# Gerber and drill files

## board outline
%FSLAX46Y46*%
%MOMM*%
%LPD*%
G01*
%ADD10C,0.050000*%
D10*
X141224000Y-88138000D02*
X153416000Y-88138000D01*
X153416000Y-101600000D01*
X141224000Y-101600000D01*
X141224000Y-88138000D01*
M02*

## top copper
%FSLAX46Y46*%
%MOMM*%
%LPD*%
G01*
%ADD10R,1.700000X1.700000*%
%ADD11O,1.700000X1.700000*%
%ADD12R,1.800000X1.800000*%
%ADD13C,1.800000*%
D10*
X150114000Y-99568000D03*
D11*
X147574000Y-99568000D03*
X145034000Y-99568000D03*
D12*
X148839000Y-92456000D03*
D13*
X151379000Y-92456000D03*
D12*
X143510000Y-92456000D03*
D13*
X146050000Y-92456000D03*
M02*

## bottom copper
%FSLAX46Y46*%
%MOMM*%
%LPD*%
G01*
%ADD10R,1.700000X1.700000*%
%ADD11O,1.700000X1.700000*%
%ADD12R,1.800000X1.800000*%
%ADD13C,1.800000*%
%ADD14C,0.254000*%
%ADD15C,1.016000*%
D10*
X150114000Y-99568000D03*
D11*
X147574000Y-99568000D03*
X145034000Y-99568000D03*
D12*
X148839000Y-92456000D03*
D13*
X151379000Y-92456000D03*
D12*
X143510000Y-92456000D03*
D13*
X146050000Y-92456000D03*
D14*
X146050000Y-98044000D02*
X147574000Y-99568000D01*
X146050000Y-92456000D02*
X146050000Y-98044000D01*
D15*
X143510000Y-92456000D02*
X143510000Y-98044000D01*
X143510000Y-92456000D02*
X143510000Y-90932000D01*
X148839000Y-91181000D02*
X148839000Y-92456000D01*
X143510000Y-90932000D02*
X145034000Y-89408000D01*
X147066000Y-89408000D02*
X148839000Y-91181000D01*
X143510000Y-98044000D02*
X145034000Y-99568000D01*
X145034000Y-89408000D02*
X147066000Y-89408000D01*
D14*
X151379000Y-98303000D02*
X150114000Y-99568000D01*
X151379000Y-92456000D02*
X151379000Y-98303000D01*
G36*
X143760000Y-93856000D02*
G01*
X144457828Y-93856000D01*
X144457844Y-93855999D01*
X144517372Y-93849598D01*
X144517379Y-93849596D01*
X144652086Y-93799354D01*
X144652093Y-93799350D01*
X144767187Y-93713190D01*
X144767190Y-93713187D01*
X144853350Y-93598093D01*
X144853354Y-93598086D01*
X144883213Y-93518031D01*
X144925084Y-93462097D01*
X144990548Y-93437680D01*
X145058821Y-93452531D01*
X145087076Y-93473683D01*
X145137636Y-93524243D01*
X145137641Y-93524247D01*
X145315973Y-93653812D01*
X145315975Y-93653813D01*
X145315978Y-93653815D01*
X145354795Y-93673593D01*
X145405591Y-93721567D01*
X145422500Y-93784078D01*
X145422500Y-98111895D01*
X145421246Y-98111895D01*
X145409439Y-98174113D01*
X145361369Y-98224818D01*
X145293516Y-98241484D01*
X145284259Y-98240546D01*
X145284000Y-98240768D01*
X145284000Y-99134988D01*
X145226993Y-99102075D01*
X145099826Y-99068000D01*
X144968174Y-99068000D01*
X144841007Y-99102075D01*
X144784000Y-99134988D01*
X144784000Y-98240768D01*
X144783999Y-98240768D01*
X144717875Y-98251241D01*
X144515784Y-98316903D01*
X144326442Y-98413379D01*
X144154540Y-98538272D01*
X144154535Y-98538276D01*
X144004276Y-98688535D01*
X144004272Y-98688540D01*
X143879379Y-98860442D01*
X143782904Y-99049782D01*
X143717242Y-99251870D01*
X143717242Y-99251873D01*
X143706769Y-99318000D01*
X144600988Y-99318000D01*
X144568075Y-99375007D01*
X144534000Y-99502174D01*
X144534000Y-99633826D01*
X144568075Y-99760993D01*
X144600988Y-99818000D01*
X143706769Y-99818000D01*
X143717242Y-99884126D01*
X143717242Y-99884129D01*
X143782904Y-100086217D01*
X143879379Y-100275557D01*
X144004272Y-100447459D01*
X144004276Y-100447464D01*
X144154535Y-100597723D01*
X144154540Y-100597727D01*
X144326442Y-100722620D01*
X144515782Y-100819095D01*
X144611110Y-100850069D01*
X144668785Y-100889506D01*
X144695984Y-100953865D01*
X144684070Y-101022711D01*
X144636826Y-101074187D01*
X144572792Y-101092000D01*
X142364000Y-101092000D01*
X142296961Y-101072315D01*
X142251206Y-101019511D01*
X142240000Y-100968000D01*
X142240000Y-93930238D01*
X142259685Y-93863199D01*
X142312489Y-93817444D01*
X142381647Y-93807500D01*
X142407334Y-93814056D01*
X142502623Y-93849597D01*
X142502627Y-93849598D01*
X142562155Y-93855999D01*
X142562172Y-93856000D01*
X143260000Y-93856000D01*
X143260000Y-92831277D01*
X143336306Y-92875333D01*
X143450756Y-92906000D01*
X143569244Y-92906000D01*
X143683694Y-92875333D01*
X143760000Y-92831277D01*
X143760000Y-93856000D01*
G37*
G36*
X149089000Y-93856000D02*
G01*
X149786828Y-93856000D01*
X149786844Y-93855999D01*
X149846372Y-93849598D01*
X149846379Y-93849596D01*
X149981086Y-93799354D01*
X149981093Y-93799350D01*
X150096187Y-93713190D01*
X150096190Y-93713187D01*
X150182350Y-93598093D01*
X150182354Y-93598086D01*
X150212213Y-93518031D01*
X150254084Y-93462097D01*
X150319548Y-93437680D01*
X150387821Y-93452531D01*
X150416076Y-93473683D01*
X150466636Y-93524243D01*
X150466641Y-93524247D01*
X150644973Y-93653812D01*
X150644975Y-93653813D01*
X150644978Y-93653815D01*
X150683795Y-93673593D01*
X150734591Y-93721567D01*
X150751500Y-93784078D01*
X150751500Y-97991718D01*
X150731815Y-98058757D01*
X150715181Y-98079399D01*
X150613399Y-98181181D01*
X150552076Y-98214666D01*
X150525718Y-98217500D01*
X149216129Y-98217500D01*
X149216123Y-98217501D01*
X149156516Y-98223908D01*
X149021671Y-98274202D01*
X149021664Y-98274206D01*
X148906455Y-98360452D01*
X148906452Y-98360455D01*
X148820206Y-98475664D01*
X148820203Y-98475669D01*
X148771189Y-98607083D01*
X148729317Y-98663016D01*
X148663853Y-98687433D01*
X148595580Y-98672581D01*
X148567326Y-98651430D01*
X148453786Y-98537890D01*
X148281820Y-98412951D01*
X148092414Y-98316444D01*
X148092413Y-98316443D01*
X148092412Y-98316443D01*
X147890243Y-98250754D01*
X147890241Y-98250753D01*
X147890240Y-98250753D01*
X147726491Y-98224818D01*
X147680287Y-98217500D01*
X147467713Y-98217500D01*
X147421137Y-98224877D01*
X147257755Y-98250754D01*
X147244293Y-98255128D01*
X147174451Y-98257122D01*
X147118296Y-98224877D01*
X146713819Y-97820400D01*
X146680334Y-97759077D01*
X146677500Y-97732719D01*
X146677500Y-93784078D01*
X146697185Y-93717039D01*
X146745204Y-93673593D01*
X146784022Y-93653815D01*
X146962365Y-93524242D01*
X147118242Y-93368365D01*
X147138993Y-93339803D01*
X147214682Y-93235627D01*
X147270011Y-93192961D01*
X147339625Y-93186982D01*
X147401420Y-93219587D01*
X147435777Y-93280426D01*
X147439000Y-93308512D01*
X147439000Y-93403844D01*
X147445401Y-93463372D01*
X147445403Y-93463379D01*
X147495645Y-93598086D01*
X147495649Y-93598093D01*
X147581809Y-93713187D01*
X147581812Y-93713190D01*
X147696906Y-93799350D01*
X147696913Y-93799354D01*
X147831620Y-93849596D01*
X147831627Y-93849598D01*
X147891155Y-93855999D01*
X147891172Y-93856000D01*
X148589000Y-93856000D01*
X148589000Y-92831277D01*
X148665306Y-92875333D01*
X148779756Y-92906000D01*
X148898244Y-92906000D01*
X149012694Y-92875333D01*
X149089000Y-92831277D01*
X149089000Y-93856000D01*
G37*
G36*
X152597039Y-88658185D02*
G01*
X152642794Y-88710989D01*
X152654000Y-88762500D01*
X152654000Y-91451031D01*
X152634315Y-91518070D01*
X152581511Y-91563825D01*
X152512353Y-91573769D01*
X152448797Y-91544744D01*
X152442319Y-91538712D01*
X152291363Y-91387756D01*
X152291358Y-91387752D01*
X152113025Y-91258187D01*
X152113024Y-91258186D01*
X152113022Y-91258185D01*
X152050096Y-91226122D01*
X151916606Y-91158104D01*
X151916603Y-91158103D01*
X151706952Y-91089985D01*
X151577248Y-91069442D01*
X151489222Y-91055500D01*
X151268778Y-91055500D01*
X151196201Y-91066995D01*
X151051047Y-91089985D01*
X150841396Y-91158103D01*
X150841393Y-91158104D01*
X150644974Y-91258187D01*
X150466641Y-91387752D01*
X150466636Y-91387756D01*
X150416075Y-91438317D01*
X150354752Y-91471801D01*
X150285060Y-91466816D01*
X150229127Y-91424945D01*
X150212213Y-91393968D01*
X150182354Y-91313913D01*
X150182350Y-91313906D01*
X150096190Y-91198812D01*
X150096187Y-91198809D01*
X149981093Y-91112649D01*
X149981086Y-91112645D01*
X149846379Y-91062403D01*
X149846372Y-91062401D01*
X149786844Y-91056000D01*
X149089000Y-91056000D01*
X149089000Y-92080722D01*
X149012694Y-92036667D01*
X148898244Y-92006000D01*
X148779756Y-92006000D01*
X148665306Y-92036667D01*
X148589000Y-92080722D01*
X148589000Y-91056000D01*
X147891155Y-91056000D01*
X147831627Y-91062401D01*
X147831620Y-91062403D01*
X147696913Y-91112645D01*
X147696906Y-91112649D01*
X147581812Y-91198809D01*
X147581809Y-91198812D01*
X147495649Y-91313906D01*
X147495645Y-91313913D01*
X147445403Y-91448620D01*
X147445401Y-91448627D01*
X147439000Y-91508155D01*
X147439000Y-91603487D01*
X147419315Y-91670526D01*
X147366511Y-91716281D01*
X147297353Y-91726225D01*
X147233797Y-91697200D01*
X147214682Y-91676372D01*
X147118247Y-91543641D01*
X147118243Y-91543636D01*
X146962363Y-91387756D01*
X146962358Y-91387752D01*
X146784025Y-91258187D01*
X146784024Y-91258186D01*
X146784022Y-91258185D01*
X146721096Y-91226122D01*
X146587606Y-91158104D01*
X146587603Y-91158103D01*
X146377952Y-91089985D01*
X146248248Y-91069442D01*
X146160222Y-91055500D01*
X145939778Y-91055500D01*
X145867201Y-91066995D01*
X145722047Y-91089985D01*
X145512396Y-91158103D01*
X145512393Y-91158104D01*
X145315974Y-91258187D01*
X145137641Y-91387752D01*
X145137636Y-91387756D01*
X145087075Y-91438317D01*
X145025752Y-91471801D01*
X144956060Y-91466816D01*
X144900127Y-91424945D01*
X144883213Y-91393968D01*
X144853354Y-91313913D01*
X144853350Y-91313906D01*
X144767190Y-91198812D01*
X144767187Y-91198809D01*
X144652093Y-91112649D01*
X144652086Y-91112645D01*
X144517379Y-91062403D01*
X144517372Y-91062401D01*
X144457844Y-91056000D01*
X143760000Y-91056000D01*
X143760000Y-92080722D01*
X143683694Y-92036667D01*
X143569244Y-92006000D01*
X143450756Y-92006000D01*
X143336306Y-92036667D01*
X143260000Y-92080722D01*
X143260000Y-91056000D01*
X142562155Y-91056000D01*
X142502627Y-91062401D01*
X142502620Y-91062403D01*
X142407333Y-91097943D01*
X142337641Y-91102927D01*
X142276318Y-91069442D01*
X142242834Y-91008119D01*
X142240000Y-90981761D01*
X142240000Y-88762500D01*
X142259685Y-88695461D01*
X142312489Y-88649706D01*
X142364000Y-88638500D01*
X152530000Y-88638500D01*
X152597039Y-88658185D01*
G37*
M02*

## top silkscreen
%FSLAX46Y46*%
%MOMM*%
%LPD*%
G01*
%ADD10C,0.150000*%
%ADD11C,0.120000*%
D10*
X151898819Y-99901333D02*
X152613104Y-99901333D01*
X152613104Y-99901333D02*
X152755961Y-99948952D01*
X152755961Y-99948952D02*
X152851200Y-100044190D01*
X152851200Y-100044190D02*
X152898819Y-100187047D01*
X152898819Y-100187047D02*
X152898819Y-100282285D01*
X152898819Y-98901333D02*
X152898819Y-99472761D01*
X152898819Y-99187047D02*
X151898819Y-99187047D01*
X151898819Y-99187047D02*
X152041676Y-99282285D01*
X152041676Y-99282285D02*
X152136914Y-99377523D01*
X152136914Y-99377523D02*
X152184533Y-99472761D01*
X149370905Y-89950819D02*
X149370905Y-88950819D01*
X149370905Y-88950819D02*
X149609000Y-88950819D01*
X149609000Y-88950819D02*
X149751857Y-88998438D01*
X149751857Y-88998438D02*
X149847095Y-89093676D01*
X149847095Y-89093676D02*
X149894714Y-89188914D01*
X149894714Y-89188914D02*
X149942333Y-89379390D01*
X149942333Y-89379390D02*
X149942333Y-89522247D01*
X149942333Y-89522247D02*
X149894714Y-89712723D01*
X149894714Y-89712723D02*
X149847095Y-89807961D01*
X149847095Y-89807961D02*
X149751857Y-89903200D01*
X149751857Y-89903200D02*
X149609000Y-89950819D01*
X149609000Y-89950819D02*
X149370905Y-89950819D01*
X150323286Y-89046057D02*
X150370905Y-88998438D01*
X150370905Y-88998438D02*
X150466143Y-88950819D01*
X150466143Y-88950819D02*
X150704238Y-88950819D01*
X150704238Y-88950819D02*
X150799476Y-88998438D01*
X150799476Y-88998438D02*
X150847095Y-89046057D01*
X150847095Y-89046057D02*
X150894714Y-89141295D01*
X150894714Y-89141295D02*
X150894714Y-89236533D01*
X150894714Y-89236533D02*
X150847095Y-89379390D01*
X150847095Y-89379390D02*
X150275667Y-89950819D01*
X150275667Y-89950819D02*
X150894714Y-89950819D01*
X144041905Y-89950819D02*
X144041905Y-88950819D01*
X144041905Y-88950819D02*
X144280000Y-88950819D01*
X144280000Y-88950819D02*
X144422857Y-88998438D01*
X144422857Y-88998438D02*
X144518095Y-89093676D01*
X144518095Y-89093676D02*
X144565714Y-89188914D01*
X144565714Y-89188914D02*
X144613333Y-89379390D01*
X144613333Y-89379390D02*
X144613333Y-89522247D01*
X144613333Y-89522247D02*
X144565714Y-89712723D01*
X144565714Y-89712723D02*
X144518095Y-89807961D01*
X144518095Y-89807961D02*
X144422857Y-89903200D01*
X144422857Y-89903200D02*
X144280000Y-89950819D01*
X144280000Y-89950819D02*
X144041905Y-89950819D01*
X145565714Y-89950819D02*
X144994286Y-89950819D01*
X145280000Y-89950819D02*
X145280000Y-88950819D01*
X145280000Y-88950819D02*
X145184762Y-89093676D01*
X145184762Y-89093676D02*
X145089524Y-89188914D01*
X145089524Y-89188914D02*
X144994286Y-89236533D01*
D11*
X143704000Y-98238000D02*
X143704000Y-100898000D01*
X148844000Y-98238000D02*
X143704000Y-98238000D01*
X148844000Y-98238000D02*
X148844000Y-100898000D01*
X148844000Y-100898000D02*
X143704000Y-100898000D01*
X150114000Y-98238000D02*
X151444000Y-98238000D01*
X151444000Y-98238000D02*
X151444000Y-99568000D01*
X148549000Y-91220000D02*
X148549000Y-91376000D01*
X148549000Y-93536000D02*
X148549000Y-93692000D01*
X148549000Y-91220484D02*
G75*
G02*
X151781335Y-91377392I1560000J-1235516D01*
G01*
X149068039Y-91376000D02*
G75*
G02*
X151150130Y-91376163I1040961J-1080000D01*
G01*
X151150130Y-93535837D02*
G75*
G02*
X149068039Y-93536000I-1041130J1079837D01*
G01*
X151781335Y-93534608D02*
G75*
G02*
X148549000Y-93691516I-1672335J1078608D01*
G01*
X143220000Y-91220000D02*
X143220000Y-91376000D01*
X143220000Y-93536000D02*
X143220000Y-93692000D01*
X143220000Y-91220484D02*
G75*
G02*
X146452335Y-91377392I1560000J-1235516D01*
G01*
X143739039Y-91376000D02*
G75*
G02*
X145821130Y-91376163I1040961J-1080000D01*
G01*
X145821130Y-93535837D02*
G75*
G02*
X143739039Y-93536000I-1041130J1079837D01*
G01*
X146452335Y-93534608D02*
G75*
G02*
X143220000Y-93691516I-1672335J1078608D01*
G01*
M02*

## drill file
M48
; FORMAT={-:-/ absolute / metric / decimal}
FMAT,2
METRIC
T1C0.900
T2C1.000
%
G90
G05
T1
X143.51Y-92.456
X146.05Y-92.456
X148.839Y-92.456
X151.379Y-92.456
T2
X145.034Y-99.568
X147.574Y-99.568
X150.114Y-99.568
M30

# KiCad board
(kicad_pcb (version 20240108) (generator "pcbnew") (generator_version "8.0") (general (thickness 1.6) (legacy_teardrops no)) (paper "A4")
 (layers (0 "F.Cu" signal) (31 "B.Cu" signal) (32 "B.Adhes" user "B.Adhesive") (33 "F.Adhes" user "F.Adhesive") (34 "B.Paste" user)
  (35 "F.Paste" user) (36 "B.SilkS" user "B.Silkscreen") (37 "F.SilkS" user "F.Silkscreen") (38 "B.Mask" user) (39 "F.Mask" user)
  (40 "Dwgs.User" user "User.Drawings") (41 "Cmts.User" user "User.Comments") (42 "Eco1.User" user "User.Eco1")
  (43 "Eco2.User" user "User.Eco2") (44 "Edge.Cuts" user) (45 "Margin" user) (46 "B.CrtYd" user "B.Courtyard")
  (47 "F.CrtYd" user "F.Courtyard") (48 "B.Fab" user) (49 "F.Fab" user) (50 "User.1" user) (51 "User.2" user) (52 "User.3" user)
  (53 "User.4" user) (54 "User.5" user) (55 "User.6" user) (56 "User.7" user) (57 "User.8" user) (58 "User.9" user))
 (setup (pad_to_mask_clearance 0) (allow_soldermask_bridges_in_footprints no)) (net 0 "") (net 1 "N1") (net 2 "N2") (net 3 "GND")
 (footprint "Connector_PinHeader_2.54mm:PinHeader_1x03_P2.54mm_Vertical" (layer "F.Cu") (at 150.114 99.568 -90)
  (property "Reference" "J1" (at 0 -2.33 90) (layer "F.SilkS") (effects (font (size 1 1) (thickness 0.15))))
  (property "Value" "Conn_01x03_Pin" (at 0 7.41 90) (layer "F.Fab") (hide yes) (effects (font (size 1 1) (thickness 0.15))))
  (fp_line (start -1.33 6.41) (end 1.33 6.41) (stroke (width 0.12) (type solid)) (layer "F.SilkS"))
  (fp_line (start -1.33 1.27) (end -1.33 6.41) (stroke (width 0.12) (type solid)) (layer "F.SilkS"))
  (fp_line (start -1.33 1.27) (end 1.33 1.27) (stroke (width 0.12) (type solid)) (layer "F.SilkS"))
  (fp_line (start 1.33 1.27) (end 1.33 6.41) (stroke (width 0.12) (type solid)) (layer "F.SilkS"))
  (fp_line (start -1.33 0) (end -1.33 -1.33) (stroke (width 0.12) (type solid)) (layer "F.SilkS"))
  (fp_line (start -1.33 -1.33) (end 0 -1.33) (stroke (width 0.12) (type solid)) (layer "F.SilkS"))
  (pad "1" thru_hole rect (at 0 0 270) (size 1.7 1.7) (drill 1) (layers "*.Cu" "*.Mask") (remove_unused_layers no) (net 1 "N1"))
  (pad "2" thru_hole oval (at 0 2.54 270) (size 1.7 1.7) (drill 1) (layers "*.Cu" "*.Mask") (remove_unused_layers no) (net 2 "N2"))
  (pad "3" thru_hole oval (at 0 5.08 270) (size 1.7 1.7) (drill 1) (layers "*.Cu" "*.Mask") (remove_unused_layers no) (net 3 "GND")))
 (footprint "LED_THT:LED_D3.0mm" (layer "F.Cu") (at 148.839 92.456)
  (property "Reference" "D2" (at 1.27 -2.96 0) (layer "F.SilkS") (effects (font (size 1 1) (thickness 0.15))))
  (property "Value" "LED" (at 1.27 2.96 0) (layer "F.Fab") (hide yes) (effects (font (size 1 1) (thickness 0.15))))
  (fp_line (start -0.29 -1.236) (end -0.29 -1.08) (stroke (width 0.12) (type solid)) (layer "F.SilkS"))
  (fp_line (start -0.29 1.08) (end -0.29 1.236) (stroke (width 0.12) (type solid)) (layer "F.SilkS"))
  (fp_arc (start -0.29 -1.235516) (mid 1.366487 -1.987659) (end 2.942335 -1.078608) (stroke (width 0.12) (type solid)) (layer "F.SilkS"))
  (fp_arc (start 0.229039 -1.08) (mid 1.270117 -1.5) (end 2.31113 -1.079837) (stroke (width 0.12) (type solid)) (layer "F.SilkS"))
  (fp_arc (start 2.31113 1.079837) (mid 1.270117 1.5) (end 0.229039 1.08) (stroke (width 0.12) (type solid)) (layer "F.SilkS"))
  (fp_arc (start 2.942335 1.078608) (mid 1.366487 1.987659) (end -0.29 1.235516) (stroke (width 0.12) (type solid)) (layer "F.SilkS"))
  (pad "1" thru_hole rect (at 0 0) (size 1.8 1.8) (drill 0.9) (layers "*.Cu" "*.Mask") (remove_unused_layers no) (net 3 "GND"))
  (pad "2" thru_hole circle (at 2.54 0) (size 1.8 1.8) (drill 0.9) (layers "*.Cu" "*.Mask") (remove_unused_layers no) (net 1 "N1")))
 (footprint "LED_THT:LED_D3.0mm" (layer "F.Cu") (at 143.51 92.456)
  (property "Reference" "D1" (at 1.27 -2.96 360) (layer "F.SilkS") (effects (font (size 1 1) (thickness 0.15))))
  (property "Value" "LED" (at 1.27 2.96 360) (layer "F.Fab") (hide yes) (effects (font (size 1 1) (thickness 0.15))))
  (fp_line (start -0.29 -1.236) (end -0.29 -1.08) (stroke (width 0.12) (type solid)) (layer "F.SilkS"))
  (fp_line (start -0.29 1.08) (end -0.29 1.236) (stroke (width 0.12) (type solid)) (layer "F.SilkS"))
  (fp_arc (start -0.29 -1.235516) (mid 1.366487 -1.987659) (end 2.942335 -1.078608) (stroke (width 0.12) (type solid)) (layer "F.SilkS"))
  (fp_arc (start 0.229039 -1.08) (mid 1.270117 -1.5) (end 2.31113 -1.079837) (stroke (width 0.12) (type solid)) (layer "F.SilkS"))
  (fp_arc (start 2.31113 1.079837) (mid 1.270117 1.5) (end 0.229039 1.08) (stroke (width 0.12) (type solid)) (layer "F.SilkS"))
  (fp_arc (start 2.942335 1.078608) (mid 1.366487 1.987659) (end -0.29 1.235516) (stroke (width 0.12) (type solid)) (layer "F.SilkS"))
  (pad "1" thru_hole rect (at 0 0) (size 1.8 1.8) (drill 0.9) (layers "*.Cu" "*.Mask") (remove_unused_layers no) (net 3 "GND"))
  (pad "2" thru_hole circle (at 2.54 0) (size 1.8 1.8) (drill 0.9) (layers "*.Cu" "*.Mask") (remove_unused_layers no) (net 2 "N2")))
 (gr_rect (start 141.224 88.138) (end 153.416 101.6) (stroke (width 0.05) (type default)) (fill none) (layer "Edge.Cuts"))
 (segment (start 146.05 98.044) (end 147.574 99.568) (width 0.254) (layer "B.Cu") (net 2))
 (segment (start 146.05 92.456) (end 146.05 98.044) (width 0.254) (layer "B.Cu") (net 2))
 (segment (start 143.51 92.456) (end 143.51 98.044) (width 1.016) (layer "B.Cu") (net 3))
 (segment (start 143.51 92.456) (end 143.51 90.932) (width 1.016) (layer "B.Cu") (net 3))
 (segment (start 148.839 91.181) (end 148.839 92.456) (width 1.016) (layer "B.Cu") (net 3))
 (segment (start 143.51 90.932) (end 145.034 89.408) (width 1.016) (layer "B.Cu") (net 3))
 (segment (start 147.066 89.408) (end 148.839 91.181) (width 1.016) (layer "B.Cu") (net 3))
 (segment (start 143.51 98.044) (end 145.034 99.568) (width 1.016) (layer "B.Cu") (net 3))
 (segment (start 145.034 89.408) (end 147.066 89.408) (width 1.016) (layer "B.Cu") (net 3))
 (segment (start 151.379 98.303) (end 150.114 99.568) (width 0.254) (layer "B.Cu") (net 1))
 (segment (start 151.379 92.456) (end 151.379 98.303) (width 0.254) (layer "B.Cu") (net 1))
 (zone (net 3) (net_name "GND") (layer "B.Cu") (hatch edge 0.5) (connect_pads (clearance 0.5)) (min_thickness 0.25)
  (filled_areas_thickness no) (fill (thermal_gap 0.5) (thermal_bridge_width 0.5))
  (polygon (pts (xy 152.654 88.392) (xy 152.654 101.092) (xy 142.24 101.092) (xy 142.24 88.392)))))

